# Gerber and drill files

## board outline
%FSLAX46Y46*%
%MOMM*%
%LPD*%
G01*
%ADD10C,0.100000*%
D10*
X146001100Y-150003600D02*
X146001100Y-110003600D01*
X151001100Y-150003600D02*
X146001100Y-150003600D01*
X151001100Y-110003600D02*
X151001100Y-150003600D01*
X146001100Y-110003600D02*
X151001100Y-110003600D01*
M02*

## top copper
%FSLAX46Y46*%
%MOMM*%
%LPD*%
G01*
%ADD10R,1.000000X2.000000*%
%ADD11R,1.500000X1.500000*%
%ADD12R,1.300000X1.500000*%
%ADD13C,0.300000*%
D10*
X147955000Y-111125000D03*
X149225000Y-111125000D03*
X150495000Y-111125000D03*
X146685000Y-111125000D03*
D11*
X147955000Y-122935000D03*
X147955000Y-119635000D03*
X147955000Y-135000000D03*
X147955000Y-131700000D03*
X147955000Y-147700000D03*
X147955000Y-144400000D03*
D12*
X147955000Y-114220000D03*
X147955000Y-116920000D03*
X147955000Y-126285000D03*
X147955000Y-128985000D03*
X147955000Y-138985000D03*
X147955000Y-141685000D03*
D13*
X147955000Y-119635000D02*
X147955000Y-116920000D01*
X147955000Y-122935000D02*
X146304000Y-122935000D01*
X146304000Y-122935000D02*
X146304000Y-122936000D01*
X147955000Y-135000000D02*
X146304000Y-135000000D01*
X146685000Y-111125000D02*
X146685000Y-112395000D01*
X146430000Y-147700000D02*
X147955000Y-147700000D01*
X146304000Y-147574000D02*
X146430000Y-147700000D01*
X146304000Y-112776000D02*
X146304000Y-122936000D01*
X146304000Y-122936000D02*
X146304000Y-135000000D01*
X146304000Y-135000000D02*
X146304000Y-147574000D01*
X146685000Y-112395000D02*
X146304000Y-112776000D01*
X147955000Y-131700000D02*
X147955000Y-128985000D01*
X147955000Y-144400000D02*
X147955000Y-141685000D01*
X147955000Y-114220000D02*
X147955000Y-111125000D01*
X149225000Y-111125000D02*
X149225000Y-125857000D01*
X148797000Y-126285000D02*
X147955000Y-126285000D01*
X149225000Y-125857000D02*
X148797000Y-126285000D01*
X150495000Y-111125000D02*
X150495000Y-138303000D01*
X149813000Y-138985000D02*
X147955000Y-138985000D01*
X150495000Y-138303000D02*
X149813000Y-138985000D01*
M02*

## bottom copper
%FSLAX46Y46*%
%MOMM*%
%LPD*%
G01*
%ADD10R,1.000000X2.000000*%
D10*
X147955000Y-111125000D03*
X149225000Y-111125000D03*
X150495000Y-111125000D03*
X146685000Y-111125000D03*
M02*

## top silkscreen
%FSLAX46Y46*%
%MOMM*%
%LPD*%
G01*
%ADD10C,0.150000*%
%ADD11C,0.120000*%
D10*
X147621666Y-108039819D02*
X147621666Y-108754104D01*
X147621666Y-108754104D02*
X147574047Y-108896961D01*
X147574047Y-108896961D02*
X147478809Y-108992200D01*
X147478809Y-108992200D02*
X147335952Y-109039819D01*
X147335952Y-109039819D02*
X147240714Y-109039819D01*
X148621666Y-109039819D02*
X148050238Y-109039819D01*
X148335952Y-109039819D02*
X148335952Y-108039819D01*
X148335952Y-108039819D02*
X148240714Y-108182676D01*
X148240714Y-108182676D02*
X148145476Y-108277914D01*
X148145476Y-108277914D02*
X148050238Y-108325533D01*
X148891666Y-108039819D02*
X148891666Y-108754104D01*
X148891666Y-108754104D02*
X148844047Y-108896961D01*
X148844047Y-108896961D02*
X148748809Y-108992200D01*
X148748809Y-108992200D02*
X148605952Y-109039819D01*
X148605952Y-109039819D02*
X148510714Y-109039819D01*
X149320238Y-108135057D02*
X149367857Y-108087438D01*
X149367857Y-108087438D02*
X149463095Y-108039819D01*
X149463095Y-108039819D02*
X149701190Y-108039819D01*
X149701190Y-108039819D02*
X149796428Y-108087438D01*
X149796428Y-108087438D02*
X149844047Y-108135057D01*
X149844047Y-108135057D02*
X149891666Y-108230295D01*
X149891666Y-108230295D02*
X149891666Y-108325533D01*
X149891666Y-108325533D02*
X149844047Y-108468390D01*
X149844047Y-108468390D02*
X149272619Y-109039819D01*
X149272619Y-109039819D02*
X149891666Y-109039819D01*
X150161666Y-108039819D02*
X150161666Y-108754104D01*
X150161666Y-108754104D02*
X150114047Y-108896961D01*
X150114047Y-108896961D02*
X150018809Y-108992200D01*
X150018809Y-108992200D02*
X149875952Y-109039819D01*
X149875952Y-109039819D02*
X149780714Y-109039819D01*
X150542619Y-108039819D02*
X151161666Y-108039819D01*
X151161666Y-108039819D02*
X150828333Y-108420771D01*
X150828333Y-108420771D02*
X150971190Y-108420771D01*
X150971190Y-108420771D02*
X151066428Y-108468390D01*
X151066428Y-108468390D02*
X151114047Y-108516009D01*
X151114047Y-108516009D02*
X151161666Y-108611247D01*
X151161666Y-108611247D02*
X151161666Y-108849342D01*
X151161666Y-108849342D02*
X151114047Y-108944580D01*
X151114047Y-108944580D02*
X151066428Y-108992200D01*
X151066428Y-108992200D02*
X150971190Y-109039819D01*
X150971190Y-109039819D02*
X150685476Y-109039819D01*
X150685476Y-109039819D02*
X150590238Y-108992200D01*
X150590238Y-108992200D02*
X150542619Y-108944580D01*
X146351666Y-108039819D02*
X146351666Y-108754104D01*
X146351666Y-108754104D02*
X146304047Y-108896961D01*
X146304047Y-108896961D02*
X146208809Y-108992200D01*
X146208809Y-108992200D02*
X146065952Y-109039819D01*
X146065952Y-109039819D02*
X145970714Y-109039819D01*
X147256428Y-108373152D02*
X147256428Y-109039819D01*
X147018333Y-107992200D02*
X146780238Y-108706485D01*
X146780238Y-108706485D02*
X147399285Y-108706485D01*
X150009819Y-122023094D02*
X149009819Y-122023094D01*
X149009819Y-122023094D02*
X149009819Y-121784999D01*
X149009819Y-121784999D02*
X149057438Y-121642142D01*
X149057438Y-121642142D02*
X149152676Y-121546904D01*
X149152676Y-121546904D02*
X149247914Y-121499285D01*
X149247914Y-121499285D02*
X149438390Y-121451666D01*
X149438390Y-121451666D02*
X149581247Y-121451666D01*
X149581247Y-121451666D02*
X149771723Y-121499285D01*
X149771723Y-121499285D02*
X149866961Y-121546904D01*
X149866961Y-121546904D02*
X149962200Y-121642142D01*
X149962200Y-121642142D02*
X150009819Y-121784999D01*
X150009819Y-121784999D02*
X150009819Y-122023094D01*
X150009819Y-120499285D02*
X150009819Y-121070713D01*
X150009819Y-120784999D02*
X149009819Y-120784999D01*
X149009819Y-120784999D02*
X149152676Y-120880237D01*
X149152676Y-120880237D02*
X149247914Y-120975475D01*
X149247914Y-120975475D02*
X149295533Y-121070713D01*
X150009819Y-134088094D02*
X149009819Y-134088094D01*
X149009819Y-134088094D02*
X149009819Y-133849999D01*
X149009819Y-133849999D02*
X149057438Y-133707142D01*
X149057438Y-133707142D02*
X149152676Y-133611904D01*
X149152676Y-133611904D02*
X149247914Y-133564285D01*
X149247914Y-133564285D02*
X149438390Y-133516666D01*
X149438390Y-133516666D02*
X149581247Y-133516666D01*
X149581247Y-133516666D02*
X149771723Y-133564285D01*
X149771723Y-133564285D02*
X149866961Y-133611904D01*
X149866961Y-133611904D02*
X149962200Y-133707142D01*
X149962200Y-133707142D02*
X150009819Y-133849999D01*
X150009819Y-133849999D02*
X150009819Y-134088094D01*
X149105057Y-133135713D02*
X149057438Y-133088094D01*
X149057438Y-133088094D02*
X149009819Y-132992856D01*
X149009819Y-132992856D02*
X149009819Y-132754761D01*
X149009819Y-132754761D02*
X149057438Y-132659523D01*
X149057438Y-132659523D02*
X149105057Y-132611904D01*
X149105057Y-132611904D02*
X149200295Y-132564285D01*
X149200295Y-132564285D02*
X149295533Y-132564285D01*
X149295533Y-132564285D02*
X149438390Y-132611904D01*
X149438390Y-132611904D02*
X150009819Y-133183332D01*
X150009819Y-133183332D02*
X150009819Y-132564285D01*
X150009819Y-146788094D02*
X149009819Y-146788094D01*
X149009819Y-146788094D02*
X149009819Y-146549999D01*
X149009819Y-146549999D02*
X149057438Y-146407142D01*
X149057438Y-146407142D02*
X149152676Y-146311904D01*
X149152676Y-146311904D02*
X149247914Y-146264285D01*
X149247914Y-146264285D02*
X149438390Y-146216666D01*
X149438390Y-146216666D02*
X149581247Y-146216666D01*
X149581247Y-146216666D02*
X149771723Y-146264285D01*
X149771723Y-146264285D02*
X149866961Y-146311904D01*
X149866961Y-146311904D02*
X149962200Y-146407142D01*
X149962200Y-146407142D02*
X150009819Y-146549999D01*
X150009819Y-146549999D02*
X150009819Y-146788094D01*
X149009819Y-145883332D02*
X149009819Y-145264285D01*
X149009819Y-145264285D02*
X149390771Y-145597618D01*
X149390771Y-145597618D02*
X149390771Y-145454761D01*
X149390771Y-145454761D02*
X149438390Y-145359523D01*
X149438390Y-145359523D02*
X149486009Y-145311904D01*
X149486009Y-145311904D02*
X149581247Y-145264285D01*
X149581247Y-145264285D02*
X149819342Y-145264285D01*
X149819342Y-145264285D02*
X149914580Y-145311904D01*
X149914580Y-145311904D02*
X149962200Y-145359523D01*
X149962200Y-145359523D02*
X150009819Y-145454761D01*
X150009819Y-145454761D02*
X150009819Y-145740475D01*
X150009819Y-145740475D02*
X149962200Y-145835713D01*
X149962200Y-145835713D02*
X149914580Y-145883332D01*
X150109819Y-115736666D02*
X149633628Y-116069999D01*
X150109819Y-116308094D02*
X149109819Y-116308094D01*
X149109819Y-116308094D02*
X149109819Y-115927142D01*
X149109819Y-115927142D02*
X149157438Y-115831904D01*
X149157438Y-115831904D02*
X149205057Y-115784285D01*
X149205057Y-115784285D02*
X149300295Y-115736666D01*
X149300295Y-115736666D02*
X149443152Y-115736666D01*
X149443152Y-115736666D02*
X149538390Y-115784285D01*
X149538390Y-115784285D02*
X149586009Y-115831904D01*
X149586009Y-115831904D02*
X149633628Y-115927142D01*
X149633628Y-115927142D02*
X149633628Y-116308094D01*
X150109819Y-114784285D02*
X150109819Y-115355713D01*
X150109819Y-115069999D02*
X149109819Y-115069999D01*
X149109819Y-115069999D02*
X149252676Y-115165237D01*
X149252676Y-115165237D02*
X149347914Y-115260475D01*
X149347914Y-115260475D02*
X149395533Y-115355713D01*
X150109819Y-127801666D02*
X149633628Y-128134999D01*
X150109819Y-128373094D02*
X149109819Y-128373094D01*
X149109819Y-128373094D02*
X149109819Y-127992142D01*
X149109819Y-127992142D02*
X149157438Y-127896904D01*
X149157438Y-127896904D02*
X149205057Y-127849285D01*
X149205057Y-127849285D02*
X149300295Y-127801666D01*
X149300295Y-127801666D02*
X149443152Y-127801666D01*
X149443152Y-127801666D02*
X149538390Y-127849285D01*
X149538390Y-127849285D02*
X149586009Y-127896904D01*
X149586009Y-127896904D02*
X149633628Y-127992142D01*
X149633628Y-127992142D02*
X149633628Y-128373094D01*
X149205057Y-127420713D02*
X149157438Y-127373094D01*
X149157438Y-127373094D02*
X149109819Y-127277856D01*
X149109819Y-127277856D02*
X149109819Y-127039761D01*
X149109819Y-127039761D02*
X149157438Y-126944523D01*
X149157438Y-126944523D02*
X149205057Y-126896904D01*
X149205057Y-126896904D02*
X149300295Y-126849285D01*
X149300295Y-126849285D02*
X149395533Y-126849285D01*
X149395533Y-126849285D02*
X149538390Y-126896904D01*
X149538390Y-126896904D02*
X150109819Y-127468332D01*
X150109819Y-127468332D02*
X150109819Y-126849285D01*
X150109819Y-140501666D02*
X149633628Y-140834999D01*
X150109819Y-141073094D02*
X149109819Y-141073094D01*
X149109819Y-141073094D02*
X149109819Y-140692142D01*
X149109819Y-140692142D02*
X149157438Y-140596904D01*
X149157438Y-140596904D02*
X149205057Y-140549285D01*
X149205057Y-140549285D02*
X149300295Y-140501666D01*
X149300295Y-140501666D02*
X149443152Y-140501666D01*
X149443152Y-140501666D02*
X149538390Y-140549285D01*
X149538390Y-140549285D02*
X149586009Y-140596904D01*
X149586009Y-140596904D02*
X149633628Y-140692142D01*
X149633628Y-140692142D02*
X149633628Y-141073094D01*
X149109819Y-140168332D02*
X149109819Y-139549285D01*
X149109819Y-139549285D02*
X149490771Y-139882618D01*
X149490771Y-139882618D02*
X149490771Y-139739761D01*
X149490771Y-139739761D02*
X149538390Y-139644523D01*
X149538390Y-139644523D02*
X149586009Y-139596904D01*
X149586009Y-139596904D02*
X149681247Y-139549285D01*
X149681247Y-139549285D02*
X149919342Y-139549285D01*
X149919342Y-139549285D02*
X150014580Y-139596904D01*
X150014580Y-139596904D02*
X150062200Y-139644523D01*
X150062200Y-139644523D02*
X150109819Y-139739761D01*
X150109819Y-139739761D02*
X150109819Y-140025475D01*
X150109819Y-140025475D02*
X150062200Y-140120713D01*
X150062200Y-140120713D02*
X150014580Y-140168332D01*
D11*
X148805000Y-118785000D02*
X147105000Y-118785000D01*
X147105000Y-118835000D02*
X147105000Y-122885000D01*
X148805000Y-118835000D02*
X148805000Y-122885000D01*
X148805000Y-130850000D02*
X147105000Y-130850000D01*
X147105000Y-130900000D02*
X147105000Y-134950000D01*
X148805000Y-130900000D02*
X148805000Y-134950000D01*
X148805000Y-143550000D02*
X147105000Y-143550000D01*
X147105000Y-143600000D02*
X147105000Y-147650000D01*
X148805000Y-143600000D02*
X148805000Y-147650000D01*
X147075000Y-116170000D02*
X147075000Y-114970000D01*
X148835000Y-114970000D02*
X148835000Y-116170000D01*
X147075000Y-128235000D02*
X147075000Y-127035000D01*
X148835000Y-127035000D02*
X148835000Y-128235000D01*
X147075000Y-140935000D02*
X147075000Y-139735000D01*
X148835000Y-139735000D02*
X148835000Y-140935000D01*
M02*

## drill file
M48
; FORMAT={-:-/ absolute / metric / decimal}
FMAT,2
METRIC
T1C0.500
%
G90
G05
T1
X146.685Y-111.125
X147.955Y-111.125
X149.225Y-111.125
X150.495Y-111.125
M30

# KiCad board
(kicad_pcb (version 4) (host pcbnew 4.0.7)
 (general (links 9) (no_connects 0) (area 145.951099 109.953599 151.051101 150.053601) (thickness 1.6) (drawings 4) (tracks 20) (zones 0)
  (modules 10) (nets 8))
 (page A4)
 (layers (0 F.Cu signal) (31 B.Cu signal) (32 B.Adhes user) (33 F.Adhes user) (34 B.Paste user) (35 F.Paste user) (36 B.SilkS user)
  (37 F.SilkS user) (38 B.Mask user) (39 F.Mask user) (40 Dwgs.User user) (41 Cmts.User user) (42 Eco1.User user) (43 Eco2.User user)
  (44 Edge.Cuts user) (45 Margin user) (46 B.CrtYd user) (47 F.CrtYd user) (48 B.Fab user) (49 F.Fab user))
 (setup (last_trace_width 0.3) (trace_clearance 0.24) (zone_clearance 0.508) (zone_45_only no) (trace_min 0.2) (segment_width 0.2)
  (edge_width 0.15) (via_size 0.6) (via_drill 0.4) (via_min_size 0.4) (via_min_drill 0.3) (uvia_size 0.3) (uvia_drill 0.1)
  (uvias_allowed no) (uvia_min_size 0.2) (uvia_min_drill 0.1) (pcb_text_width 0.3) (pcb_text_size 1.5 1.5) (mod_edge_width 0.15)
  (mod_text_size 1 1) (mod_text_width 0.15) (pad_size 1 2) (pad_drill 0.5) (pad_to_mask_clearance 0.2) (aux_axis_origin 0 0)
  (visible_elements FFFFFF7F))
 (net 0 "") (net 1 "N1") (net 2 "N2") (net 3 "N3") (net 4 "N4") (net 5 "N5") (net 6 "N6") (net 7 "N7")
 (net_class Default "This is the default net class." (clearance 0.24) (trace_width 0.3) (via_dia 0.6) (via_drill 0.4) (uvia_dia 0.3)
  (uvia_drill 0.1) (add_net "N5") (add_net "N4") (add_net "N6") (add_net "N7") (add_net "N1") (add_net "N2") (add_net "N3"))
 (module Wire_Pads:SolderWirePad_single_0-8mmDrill (layer F.Cu) (at 147.955 111.125)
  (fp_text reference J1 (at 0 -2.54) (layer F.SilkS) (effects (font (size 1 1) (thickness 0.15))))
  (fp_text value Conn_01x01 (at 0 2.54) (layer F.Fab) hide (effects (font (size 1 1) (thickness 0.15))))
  (pad 1 thru_hole rect (at 0 0) (size 1 2) (drill 0.5) (layers *.Cu *.Mask) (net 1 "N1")))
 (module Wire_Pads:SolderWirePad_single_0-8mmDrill (layer F.Cu) (at 149.225 111.125)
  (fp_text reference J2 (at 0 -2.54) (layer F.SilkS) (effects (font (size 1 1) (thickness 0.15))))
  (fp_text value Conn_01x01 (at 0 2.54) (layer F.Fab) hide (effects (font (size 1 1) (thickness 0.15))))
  (pad 1 thru_hole rect (at 0 0) (size 1 2) (drill 0.5) (layers *.Cu *.Mask) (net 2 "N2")))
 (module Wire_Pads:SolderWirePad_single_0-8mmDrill (layer F.Cu) (at 150.495 111.125)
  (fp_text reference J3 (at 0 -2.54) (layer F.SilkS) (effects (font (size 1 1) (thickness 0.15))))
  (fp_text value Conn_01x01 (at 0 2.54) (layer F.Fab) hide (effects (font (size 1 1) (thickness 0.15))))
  (pad 1 thru_hole rect (at 0 0) (size 1 2) (drill 0.5) (layers *.Cu *.Mask) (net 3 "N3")))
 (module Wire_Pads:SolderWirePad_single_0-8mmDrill (layer F.Cu) (at 146.685 111.125)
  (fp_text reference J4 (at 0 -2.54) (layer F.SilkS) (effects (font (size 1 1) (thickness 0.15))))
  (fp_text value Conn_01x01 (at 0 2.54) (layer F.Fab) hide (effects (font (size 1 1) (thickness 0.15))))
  (pad 1 thru_hole rect (at 0 0) (size 1 2) (drill 0.5) (layers *.Cu *.Mask) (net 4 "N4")))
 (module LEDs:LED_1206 (layer F.Cu) (at 147.955 121.285 270)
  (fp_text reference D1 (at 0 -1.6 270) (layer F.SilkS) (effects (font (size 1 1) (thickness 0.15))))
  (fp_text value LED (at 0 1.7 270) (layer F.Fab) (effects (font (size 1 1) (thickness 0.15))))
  (fp_line (start -2.5 -0.85) (end -2.5 0.85) (layer F.SilkS) (width 0.12))
  (fp_line (start -2.45 0.85) (end 1.6 0.85) (layer F.SilkS) (width 0.12))
  (fp_line (start -2.45 -0.85) (end 1.6 -0.85) (layer F.SilkS) (width 0.12))
  (pad 2 smd rect (at 1.65 0 90) (size 1.5 1.5) (layers F.Cu F.Paste F.Mask) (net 4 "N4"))
  (pad 1 smd rect (at -1.65 0 90) (size 1.5 1.5) (layers F.Cu F.Paste F.Mask) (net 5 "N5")))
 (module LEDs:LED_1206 (layer F.Cu) (at 147.955 133.35 270)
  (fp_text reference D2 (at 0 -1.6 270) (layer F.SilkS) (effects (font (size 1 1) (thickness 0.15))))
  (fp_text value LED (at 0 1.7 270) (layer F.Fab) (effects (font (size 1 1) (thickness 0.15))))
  (fp_line (start -2.5 -0.85) (end -2.5 0.85) (layer F.SilkS) (width 0.12))
  (fp_line (start -2.45 0.85) (end 1.6 0.85) (layer F.SilkS) (width 0.12))
  (fp_line (start -2.45 -0.85) (end 1.6 -0.85) (layer F.SilkS) (width 0.12))
  (pad 2 smd rect (at 1.65 0 90) (size 1.5 1.5) (layers F.Cu F.Paste F.Mask) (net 4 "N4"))
  (pad 1 smd rect (at -1.65 0 90) (size 1.5 1.5) (layers F.Cu F.Paste F.Mask) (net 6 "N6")))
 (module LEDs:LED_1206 (layer F.Cu) (at 147.955 146.05 270)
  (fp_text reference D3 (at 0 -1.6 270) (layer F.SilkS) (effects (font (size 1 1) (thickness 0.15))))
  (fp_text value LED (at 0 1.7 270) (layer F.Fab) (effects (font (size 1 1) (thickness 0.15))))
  (fp_line (start -2.5 -0.85) (end -2.5 0.85) (layer F.SilkS) (width 0.12))
  (fp_line (start -2.45 0.85) (end 1.6 0.85) (layer F.SilkS) (width 0.12))
  (fp_line (start -2.45 -0.85) (end 1.6 -0.85) (layer F.SilkS) (width 0.12))
  (pad 2 smd rect (at 1.65 0 90) (size 1.5 1.5) (layers F.Cu F.Paste F.Mask) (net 4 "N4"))
  (pad 1 smd rect (at -1.65 0 90) (size 1.5 1.5) (layers F.Cu F.Paste F.Mask) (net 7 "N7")))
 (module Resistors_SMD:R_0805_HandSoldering (layer F.Cu) (at 147.955 115.57 270)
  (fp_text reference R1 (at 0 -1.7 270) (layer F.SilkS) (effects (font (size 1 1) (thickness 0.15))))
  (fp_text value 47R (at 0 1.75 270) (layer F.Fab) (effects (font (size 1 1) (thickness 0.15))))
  (fp_line (start 0.6 0.88) (end -0.6 0.88) (layer F.SilkS) (width 0.12))
  (fp_line (start -0.6 -0.88) (end 0.6 -0.88) (layer F.SilkS) (width 0.12))
  (pad 1 smd rect (at -1.35 0 270) (size 1.5 1.3) (layers F.Cu F.Paste F.Mask) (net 1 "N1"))
  (pad 2 smd rect (at 1.35 0 270) (size 1.5 1.3) (layers F.Cu F.Paste F.Mask) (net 5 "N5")))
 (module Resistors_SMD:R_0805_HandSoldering (layer F.Cu) (at 147.955 127.635 270)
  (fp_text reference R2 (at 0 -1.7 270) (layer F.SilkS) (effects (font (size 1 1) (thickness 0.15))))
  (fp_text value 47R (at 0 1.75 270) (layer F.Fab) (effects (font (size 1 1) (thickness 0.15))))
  (fp_line (start 0.6 0.88) (end -0.6 0.88) (layer F.SilkS) (width 0.12))
  (fp_line (start -0.6 -0.88) (end 0.6 -0.88) (layer F.SilkS) (width 0.12))
  (pad 1 smd rect (at -1.35 0 270) (size 1.5 1.3) (layers F.Cu F.Paste F.Mask) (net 2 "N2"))
  (pad 2 smd rect (at 1.35 0 270) (size 1.5 1.3) (layers F.Cu F.Paste F.Mask) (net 6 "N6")))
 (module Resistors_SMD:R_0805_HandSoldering (layer F.Cu) (at 147.955 140.335 270)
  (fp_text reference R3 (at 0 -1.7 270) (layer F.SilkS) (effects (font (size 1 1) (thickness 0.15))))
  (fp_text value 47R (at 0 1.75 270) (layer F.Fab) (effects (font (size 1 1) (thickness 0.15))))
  (fp_line (start 0.6 0.88) (end -0.6 0.88) (layer F.SilkS) (width 0.12))
  (fp_line (start -0.6 -0.88) (end 0.6 -0.88) (layer F.SilkS) (width 0.12))
  (pad 1 smd rect (at -1.35 0 270) (size 1.5 1.3) (layers F.Cu F.Paste F.Mask) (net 3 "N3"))
  (pad 2 smd rect (at 1.35 0 270) (size 1.5 1.3) (layers F.Cu F.Paste F.Mask) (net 7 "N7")))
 (gr_line (start 146.0011 150.0036) (end 146.0011 110.0036) (layer Edge.Cuts) (width 0.1))
 (gr_line (start 151.0011 150.0036) (end 146.0011 150.0036) (layer Edge.Cuts) (width 0.1))
 (gr_line (start 151.0011 110.0036) (end 151.0011 150.0036) (layer Edge.Cuts) (width 0.1))
 (gr_line (start 146.0011 110.0036) (end 151.0011 110.0036) (layer Edge.Cuts) (width 0.1))
 (segment (start 147.955 119.635) (end 147.955 116.92) (width 0.3) (layer F.Cu) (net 5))
 (segment (start 147.955 122.935) (end 146.304 122.935) (width 0.3) (layer F.Cu) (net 4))
 (segment (start 146.304 122.935) (end 146.304 122.936) (width 0.3) (layer F.Cu) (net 4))
 (segment (start 147.955 135) (end 146.304 135) (width 0.3) (layer F.Cu) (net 4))
 (segment (start 146.685 111.125) (end 146.685 112.395) (width 0.3) (layer F.Cu) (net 4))
 (segment (start 146.43 147.7) (end 147.955 147.7) (width 0.3) (layer F.Cu) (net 4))
 (segment (start 146.304 147.574) (end 146.43 147.7) (width 0.3) (layer F.Cu) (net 4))
 (segment (start 146.304 112.776) (end 146.304 122.936) (width 0.3) (layer F.Cu) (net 4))
 (segment (start 146.304 122.936) (end 146.304 135) (width 0.3) (layer F.Cu) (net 4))
 (segment (start 146.304 135) (end 146.304 147.574) (width 0.3) (layer F.Cu) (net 4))
 (segment (start 146.685 112.395) (end 146.304 112.776) (width 0.3) (layer F.Cu) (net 4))
 (segment (start 147.955 131.7) (end 147.955 128.985) (width 0.3) (layer F.Cu) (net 6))
 (segment (start 147.955 144.4) (end 147.955 141.685) (width 0.3) (layer F.Cu) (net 7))
 (segment (start 147.955 114.22) (end 147.955 111.125) (width 0.3) (layer F.Cu) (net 1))
 (segment (start 149.225 111.125) (end 149.225 125.857) (width 0.3) (layer F.Cu) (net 2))
 (segment (start 148.797 126.285) (end 147.955 126.285) (width 0.3) (layer F.Cu) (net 2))
 (segment (start 149.225 125.857) (end 148.797 126.285) (width 0.3) (layer F.Cu) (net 2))
 (segment (start 150.495 111.125) (end 150.495 138.303) (width 0.3) (layer F.Cu) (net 3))
 (segment (start 149.813 138.985) (end 147.955 138.985) (width 0.3) (layer F.Cu) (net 3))
 (segment (start 150.495 138.303) (end 149.813 138.985) (width 0.3) (layer F.Cu) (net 3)))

